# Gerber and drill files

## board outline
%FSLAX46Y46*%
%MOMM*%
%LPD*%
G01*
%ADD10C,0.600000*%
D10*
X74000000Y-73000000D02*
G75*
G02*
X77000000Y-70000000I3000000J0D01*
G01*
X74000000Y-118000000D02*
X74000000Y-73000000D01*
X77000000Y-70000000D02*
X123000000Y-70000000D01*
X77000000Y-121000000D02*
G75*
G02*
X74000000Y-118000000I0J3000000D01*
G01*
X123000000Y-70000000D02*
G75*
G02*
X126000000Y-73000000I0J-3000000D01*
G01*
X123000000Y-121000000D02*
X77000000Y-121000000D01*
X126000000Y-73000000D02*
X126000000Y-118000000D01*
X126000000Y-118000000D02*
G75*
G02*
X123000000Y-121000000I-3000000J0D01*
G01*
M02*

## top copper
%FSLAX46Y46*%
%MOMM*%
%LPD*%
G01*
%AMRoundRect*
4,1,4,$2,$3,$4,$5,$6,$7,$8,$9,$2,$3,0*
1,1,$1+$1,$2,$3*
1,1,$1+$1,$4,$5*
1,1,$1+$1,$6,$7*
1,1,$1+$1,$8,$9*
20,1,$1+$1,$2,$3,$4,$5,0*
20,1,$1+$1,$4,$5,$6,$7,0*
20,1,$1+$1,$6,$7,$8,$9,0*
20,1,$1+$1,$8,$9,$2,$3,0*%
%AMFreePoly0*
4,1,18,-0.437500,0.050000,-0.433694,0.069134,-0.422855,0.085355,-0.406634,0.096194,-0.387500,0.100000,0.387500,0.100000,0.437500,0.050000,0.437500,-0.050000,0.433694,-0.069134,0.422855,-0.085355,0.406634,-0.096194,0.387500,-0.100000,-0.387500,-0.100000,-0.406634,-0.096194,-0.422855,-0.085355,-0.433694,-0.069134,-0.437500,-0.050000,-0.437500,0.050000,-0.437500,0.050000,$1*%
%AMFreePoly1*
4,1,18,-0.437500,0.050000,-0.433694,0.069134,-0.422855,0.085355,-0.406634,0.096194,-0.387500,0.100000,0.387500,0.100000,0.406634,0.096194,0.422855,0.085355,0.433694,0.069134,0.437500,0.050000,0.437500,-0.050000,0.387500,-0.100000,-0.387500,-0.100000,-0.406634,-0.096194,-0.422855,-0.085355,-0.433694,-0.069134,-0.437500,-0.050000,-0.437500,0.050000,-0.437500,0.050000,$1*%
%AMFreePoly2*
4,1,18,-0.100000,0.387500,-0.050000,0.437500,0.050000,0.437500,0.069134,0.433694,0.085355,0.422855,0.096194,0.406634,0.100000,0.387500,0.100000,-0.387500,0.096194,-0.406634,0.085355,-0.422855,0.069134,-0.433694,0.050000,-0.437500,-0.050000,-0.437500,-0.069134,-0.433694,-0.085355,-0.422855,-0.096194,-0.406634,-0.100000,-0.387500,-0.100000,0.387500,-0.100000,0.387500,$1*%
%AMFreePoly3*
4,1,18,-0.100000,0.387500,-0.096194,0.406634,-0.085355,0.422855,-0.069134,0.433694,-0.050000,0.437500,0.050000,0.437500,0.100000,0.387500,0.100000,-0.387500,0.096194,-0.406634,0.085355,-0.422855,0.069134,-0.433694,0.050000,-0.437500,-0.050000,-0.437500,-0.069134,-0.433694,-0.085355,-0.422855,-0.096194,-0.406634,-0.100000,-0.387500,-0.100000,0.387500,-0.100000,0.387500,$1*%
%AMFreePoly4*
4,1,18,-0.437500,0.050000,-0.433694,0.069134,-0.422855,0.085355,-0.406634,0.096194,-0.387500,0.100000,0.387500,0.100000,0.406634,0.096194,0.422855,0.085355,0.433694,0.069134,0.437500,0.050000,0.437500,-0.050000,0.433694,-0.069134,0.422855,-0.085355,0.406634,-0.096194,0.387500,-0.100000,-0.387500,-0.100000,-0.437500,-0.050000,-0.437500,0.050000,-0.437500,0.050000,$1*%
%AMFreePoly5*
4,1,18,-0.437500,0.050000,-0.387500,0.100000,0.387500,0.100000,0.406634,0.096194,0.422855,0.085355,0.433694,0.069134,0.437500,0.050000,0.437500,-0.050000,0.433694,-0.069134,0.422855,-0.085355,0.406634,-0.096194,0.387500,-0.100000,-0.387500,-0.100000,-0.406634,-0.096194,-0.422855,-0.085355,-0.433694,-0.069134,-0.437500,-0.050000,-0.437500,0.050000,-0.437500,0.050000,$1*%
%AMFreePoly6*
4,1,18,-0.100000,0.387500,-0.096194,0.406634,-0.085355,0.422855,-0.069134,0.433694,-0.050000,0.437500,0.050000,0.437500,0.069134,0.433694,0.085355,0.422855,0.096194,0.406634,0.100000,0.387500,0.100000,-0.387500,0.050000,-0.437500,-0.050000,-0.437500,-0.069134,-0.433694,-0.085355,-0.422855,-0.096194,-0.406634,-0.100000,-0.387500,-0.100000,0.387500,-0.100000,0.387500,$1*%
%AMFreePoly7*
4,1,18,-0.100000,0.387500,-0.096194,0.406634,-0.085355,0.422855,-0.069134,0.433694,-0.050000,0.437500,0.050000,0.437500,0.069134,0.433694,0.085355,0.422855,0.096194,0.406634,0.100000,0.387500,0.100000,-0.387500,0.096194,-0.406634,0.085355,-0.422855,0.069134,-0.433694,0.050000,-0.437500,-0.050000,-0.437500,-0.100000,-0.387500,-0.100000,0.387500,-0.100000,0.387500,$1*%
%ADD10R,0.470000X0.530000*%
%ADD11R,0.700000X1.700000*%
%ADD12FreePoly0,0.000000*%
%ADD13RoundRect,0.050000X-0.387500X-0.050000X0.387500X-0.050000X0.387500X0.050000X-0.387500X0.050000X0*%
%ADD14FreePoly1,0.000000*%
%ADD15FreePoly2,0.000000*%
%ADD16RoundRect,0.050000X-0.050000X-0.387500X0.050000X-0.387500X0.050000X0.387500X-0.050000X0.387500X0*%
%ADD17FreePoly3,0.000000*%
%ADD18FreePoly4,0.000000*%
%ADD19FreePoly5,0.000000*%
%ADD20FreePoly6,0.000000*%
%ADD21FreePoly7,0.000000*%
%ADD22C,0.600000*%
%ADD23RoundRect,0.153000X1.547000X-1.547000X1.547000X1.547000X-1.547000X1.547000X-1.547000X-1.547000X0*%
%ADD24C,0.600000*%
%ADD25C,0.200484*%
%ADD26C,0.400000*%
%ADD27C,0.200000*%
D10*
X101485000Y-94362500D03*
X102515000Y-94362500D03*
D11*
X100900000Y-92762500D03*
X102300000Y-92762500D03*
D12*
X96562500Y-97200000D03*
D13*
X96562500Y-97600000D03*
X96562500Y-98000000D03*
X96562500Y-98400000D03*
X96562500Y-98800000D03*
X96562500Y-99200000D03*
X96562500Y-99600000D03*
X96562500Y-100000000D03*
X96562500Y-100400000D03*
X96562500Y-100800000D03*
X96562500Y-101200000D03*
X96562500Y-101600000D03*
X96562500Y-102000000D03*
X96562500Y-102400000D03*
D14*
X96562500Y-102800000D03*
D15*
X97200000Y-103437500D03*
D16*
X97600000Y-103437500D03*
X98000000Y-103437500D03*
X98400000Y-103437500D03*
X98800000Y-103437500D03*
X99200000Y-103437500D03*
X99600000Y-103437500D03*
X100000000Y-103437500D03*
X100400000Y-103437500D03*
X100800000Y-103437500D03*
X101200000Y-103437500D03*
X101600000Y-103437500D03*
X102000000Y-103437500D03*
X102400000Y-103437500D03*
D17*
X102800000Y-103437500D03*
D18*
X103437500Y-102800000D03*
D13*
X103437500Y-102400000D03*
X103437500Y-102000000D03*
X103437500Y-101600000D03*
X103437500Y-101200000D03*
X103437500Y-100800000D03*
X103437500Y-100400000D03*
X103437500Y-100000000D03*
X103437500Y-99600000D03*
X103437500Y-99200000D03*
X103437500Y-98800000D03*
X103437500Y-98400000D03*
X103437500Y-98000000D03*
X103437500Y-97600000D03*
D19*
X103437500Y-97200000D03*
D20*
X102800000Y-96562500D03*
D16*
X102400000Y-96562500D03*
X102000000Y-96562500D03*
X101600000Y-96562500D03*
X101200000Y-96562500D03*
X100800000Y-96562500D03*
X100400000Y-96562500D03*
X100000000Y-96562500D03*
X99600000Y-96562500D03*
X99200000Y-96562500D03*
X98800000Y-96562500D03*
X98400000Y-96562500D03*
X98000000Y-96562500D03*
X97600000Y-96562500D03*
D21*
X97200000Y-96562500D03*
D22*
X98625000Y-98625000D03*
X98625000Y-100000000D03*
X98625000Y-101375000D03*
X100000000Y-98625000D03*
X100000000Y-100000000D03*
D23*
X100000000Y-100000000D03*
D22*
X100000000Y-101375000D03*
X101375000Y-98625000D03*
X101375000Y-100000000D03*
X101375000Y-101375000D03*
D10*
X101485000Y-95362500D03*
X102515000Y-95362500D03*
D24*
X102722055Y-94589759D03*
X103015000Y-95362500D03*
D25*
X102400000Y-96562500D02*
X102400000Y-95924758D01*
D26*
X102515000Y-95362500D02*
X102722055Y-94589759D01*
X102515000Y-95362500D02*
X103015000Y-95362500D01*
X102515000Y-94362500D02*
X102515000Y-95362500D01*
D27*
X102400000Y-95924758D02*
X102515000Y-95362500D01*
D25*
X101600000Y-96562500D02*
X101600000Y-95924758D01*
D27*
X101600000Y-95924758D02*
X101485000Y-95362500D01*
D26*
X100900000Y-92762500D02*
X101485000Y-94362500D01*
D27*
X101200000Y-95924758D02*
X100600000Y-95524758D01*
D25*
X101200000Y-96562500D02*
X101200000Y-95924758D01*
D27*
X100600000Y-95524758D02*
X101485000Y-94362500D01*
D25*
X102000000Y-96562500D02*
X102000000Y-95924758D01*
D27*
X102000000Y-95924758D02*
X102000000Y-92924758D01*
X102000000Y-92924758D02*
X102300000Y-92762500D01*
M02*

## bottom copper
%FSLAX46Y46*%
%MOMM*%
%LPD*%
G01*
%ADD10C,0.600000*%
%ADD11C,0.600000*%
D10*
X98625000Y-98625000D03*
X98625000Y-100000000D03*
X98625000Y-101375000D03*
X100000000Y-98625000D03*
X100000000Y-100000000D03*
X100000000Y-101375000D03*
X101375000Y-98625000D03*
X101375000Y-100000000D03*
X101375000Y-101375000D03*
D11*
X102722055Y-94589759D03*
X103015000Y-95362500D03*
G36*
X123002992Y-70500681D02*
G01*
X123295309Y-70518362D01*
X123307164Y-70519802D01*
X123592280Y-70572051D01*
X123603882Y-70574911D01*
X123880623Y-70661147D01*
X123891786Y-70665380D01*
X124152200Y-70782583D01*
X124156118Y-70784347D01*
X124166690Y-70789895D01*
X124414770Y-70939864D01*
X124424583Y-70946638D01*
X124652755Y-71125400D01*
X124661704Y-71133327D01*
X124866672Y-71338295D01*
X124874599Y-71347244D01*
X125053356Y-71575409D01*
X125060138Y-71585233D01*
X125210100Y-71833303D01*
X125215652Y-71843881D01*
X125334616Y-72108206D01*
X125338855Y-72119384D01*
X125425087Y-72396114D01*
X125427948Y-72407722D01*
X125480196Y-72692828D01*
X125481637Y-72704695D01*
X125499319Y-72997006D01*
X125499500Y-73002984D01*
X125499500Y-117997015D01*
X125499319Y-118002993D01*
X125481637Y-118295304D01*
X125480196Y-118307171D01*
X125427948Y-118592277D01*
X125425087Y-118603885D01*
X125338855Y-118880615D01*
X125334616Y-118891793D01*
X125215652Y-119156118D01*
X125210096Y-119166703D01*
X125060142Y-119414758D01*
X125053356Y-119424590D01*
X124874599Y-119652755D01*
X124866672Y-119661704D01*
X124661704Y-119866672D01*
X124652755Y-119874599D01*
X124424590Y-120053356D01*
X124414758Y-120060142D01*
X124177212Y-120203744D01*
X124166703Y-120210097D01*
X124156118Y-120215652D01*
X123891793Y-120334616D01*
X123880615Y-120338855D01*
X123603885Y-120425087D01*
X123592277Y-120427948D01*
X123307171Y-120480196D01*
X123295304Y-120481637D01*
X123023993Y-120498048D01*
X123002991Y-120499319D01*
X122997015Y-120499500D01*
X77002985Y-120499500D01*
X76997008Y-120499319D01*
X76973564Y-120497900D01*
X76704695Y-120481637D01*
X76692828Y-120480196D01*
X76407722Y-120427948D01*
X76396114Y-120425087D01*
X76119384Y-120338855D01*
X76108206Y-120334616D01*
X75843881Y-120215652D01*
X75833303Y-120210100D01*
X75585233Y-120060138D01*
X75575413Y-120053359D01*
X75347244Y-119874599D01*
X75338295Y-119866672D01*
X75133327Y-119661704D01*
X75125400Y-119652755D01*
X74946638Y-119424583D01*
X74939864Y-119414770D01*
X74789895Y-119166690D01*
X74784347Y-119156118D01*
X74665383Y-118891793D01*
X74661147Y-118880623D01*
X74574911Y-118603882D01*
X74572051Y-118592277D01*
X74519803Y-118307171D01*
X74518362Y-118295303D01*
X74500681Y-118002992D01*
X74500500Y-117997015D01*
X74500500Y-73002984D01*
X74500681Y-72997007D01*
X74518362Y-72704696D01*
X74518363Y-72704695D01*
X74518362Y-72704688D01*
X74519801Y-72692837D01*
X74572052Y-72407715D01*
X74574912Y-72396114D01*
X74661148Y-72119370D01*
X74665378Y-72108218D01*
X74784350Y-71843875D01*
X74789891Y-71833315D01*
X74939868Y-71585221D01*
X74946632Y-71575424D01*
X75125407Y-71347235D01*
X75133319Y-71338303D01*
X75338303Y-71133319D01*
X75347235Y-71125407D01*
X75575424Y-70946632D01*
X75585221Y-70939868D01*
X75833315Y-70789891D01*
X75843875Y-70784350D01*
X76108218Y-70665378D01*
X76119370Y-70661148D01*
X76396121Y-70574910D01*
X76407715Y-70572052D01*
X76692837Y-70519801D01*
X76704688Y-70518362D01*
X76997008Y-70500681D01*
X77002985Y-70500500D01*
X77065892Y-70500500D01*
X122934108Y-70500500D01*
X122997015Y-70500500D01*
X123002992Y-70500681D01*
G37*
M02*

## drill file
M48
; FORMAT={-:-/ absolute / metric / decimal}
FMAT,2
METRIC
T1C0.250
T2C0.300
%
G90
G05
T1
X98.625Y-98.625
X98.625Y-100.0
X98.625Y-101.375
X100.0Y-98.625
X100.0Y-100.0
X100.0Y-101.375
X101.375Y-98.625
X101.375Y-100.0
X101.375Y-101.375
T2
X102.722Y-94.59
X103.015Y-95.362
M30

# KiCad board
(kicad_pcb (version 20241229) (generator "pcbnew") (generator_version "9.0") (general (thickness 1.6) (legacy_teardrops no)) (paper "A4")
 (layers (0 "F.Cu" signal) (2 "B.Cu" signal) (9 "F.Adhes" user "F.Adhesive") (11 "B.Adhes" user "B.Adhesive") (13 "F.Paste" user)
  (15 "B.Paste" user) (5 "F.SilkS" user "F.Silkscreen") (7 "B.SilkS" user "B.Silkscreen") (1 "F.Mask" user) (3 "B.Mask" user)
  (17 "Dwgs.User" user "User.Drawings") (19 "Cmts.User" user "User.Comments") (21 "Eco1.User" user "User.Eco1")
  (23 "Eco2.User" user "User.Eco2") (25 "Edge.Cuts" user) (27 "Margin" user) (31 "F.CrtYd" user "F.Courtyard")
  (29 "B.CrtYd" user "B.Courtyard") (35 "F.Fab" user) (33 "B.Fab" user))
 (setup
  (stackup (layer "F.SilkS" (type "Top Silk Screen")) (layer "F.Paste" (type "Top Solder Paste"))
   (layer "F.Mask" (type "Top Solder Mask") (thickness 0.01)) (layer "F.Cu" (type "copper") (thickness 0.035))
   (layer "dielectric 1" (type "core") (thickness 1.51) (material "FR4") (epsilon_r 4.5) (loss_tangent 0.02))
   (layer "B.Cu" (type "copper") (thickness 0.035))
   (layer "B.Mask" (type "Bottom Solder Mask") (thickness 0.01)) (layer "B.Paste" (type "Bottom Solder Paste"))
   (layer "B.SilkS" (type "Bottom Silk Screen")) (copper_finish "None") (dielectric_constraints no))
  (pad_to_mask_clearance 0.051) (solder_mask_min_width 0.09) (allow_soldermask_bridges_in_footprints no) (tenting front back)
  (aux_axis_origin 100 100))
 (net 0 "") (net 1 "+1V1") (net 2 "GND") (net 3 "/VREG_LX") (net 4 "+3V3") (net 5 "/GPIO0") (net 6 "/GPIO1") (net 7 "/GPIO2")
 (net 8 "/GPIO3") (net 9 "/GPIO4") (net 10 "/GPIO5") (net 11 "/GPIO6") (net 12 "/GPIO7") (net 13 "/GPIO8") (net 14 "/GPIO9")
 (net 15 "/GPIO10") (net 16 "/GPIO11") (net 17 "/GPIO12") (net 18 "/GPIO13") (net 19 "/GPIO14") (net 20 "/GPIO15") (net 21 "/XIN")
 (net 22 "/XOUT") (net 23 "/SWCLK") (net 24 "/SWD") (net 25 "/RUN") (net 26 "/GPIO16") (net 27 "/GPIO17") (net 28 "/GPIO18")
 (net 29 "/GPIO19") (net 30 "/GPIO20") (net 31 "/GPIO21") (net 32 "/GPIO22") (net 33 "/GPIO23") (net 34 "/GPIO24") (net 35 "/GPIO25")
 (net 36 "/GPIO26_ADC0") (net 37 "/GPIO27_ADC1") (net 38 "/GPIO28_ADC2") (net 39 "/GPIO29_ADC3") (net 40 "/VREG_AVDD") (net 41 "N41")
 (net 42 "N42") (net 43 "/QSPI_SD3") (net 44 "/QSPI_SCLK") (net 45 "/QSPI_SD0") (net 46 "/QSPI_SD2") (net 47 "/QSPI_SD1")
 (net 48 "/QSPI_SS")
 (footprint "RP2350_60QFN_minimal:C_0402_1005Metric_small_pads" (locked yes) (layer "F.Cu") (at 102 94.3625)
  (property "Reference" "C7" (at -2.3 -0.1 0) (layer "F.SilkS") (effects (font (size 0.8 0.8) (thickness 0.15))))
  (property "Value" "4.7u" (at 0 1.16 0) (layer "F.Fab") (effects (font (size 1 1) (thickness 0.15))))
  (pad "1" smd rect (at -0.515 0) (size 0.47 0.53) (layers "F.Cu" "F.Mask" "F.Paste") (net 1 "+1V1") (clearance 0.125))
  (pad "2" smd rect (at 0.515 0) (size 0.47 0.53) (layers "F.Cu" "F.Mask" "F.Paste") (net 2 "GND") (clearance 0.125)))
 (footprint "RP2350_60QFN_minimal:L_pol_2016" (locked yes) (layer "F.Cu") (at 101.6 92.7625)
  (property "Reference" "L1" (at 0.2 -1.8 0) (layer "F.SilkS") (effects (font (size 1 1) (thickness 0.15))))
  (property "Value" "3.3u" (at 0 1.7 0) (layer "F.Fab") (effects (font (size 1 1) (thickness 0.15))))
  (pad "1" smd rect (at -0.7 0) (size 0.7 1.7) (layers "F.Cu" "F.Mask" "F.Paste") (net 1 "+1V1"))
  (pad "2" smd rect (at 0.7 0) (size 0.7 1.7) (layers "F.Cu" "F.Mask" "F.Paste") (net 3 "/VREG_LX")))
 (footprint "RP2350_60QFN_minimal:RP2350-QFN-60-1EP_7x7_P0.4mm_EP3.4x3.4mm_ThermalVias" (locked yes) (layer "F.Cu") (at 100 100)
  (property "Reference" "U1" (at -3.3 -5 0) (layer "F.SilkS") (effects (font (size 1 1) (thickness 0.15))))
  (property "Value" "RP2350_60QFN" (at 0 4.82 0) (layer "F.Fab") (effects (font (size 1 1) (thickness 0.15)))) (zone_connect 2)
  (pad "" smd roundrect (at -0.7 -0.7) (size 1.2 1.2) (layers "F.Paste") (roundrect_rratio 0.2083333333) (zone_connect 2))
  (pad "" smd roundrect (at -0.7 0.7) (size 1.2 1.2) (layers "F.Paste") (roundrect_rratio 0.2083333333) (zone_connect 2))
  (pad "" smd roundrect (at 0.7 -0.7) (size 1.2 1.2) (layers "F.Paste") (roundrect_rratio 0.2083333333) (zone_connect 2))
  (pad "" smd roundrect (at 0.7 0.7) (size 1.2 1.2) (layers "F.Paste") (roundrect_rratio 0.2083333333) (zone_connect 2))
  (pad "1" smd roundrect (at -3.4375 -2.8) (size 0.875 0.2) (layers "F.Cu" "F.Mask" "F.Paste") (roundrect_rratio 0.25) (chamfer_ratio 0.25)
   (chamfer top_right) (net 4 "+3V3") (zone_connect 2))
  (pad "2" smd roundrect (at -3.4375 -2.4) (size 0.875 0.2) (layers "F.Cu" "F.Mask" "F.Paste") (roundrect_rratio 0.25) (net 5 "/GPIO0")
   (zone_connect 2))
  (pad "3" smd roundrect (at -3.4375 -2) (size 0.875 0.2) (layers "F.Cu" "F.Mask" "F.Paste") (roundrect_rratio 0.25) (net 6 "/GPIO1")
   (zone_connect 2))
  (pad "4" smd roundrect (at -3.4375 -1.6) (size 0.875 0.2) (layers "F.Cu" "F.Mask" "F.Paste") (roundrect_rratio 0.25) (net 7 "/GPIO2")
   (zone_connect 2))
  (pad "5" smd roundrect (at -3.4375 -1.2) (size 0.875 0.2) (layers "F.Cu" "F.Mask" "F.Paste") (roundrect_rratio 0.25) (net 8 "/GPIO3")
   (zone_connect 2))
  (pad "6" smd roundrect (at -3.4375 -0.8) (size 0.875 0.2) (layers "F.Cu" "F.Mask" "F.Paste") (roundrect_rratio 0.25) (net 1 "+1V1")
   (zone_connect 2))
  (pad "7" smd roundrect (at -3.4375 -0.4) (size 0.875 0.2) (layers "F.Cu" "F.Mask" "F.Paste") (roundrect_rratio 0.25) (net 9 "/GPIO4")
   (zone_connect 2))
  (pad "8" smd roundrect (at -3.4375 0) (size 0.875 0.2) (layers "F.Cu" "F.Mask" "F.Paste") (roundrect_rratio 0.25) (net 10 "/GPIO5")
   (zone_connect 2))
  (pad "9" smd roundrect (at -3.4375 0.4) (size 0.875 0.2) (layers "F.Cu" "F.Mask" "F.Paste") (roundrect_rratio 0.25) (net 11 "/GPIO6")
   (zone_connect 2))
  (pad "10" smd roundrect (at -3.4375 0.8) (size 0.875 0.2) (layers "F.Cu" "F.Mask" "F.Paste") (roundrect_rratio 0.25) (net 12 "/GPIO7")
   (zone_connect 2))
  (pad "11" smd roundrect (at -3.4375 1.2) (size 0.875 0.2) (layers "F.Cu" "F.Mask" "F.Paste") (roundrect_rratio 0.25) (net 4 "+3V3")
   (zone_connect 2))
  (pad "12" smd roundrect (at -3.4375 1.6) (size 0.875 0.2) (layers "F.Cu" "F.Mask" "F.Paste") (roundrect_rratio 0.25) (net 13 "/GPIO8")
   (zone_connect 2))
  (pad "13" smd roundrect (at -3.4375 2) (size 0.875 0.2) (layers "F.Cu" "F.Mask" "F.Paste") (roundrect_rratio 0.25) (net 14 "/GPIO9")
   (zone_connect 2))
  (pad "14" smd roundrect (at -3.4375 2.4) (size 0.875 0.2) (layers "F.Cu" "F.Mask" "F.Paste") (roundrect_rratio 0.25) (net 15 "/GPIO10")
   (zone_connect 2))
  (pad "15" smd roundrect (at -3.4375 2.8) (size 0.875 0.2) (layers "F.Cu" "F.Mask" "F.Paste") (roundrect_rratio 0.25) (chamfer_ratio 0.25)
   (chamfer bottom_right) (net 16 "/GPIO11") (zone_connect 2))
  (pad "16" smd roundrect (at -2.8 3.4375) (size 0.2 0.875) (layers "F.Cu" "F.Mask" "F.Paste") (roundrect_rratio 0.25) (chamfer_ratio 0.25)
   (chamfer top_left) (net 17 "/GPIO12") (zone_connect 2))
  (pad "17" smd roundrect (at -2.4 3.4375) (size 0.2 0.875) (layers "F.Cu" "F.Mask" "F.Paste") (roundrect_rratio 0.25) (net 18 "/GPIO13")
   (zone_connect 2))
  (pad "18" smd roundrect (at -2 3.4375) (size 0.2 0.875) (layers "F.Cu" "F.Mask" "F.Paste") (roundrect_rratio 0.25) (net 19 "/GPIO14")
   (zone_connect 2))
  (pad "19" smd roundrect (at -1.6 3.4375) (size 0.2 0.875) (layers "F.Cu" "F.Mask" "F.Paste") (roundrect_rratio 0.25) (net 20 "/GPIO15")
   (zone_connect 2))
  (pad "20" smd roundrect (at -1.2 3.4375) (size 0.2 0.875) (layers "F.Cu" "F.Mask" "F.Paste") (roundrect_rratio 0.25) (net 4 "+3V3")
   (zone_connect 2))
  (pad "21" smd roundrect (at -0.8 3.4375) (size 0.2 0.875) (layers "F.Cu" "F.Mask" "F.Paste") (roundrect_rratio 0.25) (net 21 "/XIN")
   (zone_connect 2))
  (pad "22" smd roundrect (at -0.4 3.4375) (size 0.2 0.875) (layers "F.Cu" "F.Mask" "F.Paste") (roundrect_rratio 0.25) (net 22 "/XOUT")
   (zone_connect 2))
  (pad "23" smd roundrect (at 0 3.4375) (size 0.2 0.875) (layers "F.Cu" "F.Mask" "F.Paste") (roundrect_rratio 0.25) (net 1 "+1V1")
   (zone_connect 2))
  (pad "24" smd roundrect (at 0.4 3.4375) (size 0.2 0.875) (layers "F.Cu" "F.Mask" "F.Paste") (roundrect_rratio 0.25) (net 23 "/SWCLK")
   (zone_connect 2))
  (pad "25" smd roundrect (at 0.8 3.4375) (size 0.2 0.875) (layers "F.Cu" "F.Mask" "F.Paste") (roundrect_rratio 0.25) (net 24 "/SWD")
   (zone_connect 2))
  (pad "26" smd roundrect (at 1.2 3.4375) (size 0.2 0.875) (layers "F.Cu" "F.Mask" "F.Paste") (roundrect_rratio 0.25) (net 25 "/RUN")
   (zone_connect 2))
  (pad "27" smd roundrect (at 1.6 3.4375) (size 0.2 0.875) (layers "F.Cu" "F.Mask" "F.Paste") (roundrect_rratio 0.25) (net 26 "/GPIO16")
   (zone_connect 2))
  (pad "28" smd roundrect (at 2 3.4375) (size 0.2 0.875) (layers "F.Cu" "F.Mask" "F.Paste") (roundrect_rratio 0.25) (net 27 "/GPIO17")
   (zone_connect 2))
  (pad "29" smd roundrect (at 2.4 3.4375) (size 0.2 0.875) (layers "F.Cu" "F.Mask" "F.Paste") (roundrect_rratio 0.25) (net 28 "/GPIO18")
   (zone_connect 2))
  (pad "30" smd roundrect (at 2.8 3.4375) (size 0.2 0.875) (layers "F.Cu" "F.Mask" "F.Paste") (roundrect_rratio 0.25) (chamfer_ratio 0.25)
   (chamfer top_right) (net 4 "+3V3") (zone_connect 2))
  (pad "31" smd roundrect (at 3.4375 2.8) (size 0.875 0.2) (layers "F.Cu" "F.Mask" "F.Paste") (roundrect_rratio 0.25) (chamfer_ratio 0.25)
   (chamfer bottom_left) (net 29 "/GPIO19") (zone_connect 2))
  (pad "32" smd roundrect (at 3.4375 2.4) (size 0.875 0.2) (layers "F.Cu" "F.Mask" "F.Paste") (roundrect_rratio 0.25) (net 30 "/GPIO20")
   (zone_connect 2))
  (pad "33" smd roundrect (at 3.4375 2) (size 0.875 0.2) (layers "F.Cu" "F.Mask" "F.Paste") (roundrect_rratio 0.25) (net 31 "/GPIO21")
   (zone_connect 2))
  (pad "34" smd roundrect (at 3.4375 1.6) (size 0.875 0.2) (layers "F.Cu" "F.Mask" "F.Paste") (roundrect_rratio 0.25) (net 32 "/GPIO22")
   (zone_connect 2))
  (pad "35" smd roundrect (at 3.4375 1.2) (size 0.875 0.2) (layers "F.Cu" "F.Mask" "F.Paste") (roundrect_rratio 0.25) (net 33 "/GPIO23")
   (zone_connect 2))
  (pad "36" smd roundrect (at 3.4375 0.8) (size 0.875 0.2) (layers "F.Cu" "F.Mask" "F.Paste") (roundrect_rratio 0.25) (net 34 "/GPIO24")
   (zone_connect 2))
  (pad "37" smd roundrect (at 3.4375 0.4) (size 0.875 0.2) (layers "F.Cu" "F.Mask" "F.Paste") (roundrect_rratio 0.25) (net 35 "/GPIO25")
   (zone_connect 2))
  (pad "38" smd roundrect (at 3.4375 0) (size 0.875 0.2) (layers "F.Cu" "F.Mask" "F.Paste") (roundrect_rratio 0.25) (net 4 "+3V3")
   (zone_connect 2))
  (pad "39" smd roundrect (at 3.4375 -0.4) (size 0.875 0.2) (layers "F.Cu" "F.Mask" "F.Paste") (roundrect_rratio 0.25) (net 1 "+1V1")
   (zone_connect 2))
  (pad "40" smd roundrect (at 3.4375 -0.8) (size 0.875 0.2) (layers "F.Cu" "F.Mask" "F.Paste") (roundrect_rratio 0.25)
   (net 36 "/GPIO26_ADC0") (zone_connect 2))
  (pad "41" smd roundrect (at 3.4375 -1.2) (size 0.875 0.2) (layers "F.Cu" "F.Mask" "F.Paste") (roundrect_rratio 0.25)
   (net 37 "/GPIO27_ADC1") (zone_connect 2))
  (pad "42" smd roundrect (at 3.4375 -1.6) (size 0.875 0.2) (layers "F.Cu" "F.Mask" "F.Paste") (roundrect_rratio 0.25)
   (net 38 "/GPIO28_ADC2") (zone_connect 2))
  (pad "43" smd roundrect (at 3.4375 -2) (size 0.875 0.2) (layers "F.Cu" "F.Mask" "F.Paste") (roundrect_rratio 0.25) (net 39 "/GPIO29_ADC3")
   (zone_connect 2))
  (pad "44" smd roundrect (at 3.4375 -2.4) (size 0.875 0.2) (layers "F.Cu" "F.Mask" "F.Paste") (roundrect_rratio 0.25) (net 4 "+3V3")
   (zone_connect 2))
  (pad "45" smd roundrect (at 3.4375 -2.8) (size 0.875 0.2) (layers "F.Cu" "F.Mask" "F.Paste") (roundrect_rratio 0.25) (chamfer_ratio 0.25)
   (chamfer top_left) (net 4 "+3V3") (zone_connect 2))
  (pad "46" smd roundrect (at 2.8 -3.4375) (size 0.2 0.875) (layers "F.Cu" "F.Mask" "F.Paste") (roundrect_rratio 0.25) (chamfer_ratio 0.25)
   (chamfer bottom_right) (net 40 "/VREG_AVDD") (zone_connect 2))
  (pad "47" smd roundrect (at 2.4 -3.4375) (size 0.2 0.875) (layers "F.Cu" "F.Mask" "F.Paste") (roundrect_rratio 0.25) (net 2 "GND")
   (zone_connect 2))
  (pad "48" smd roundrect (at 2 -3.4375) (size 0.2 0.875) (layers "F.Cu" "F.Mask" "F.Paste") (roundrect_rratio 0.25) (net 3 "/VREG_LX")
   (zone_connect 2))
  (pad "49" smd roundrect (at 1.6 -3.4375) (size 0.2 0.875) (layers "F.Cu" "F.Mask" "F.Paste") (roundrect_rratio 0.25) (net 4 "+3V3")
   (zone_connect 2))
  (pad "50" smd roundrect (at 1.2 -3.4375) (size 0.2 0.875) (layers "F.Cu" "F.Mask" "F.Paste") (roundrect_rratio 0.25) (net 1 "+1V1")
   (zone_connect 2))
  (pad "51" smd roundrect (at 0.8 -3.4375) (size 0.2 0.875) (layers "F.Cu" "F.Mask" "F.Paste") (roundrect_rratio 0.25) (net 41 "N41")
   (zone_connect 2))
  (pad "52" smd roundrect (at 0.4 -3.4375) (size 0.2 0.875) (layers "F.Cu" "F.Mask" "F.Paste") (roundrect_rratio 0.25) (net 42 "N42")
   (zone_connect 2))
  (pad "53" smd roundrect (at 0 -3.4375) (size 0.2 0.875) (layers "F.Cu" "F.Mask" "F.Paste") (roundrect_rratio 0.25) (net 4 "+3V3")
   (zone_connect 2))
  (pad "54" smd roundrect (at -0.4 -3.4375) (size 0.2 0.875) (layers "F.Cu" "F.Mask" "F.Paste") (roundrect_rratio 0.25) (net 4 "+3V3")
   (zone_connect 2))
  (pad "55" smd roundrect (at -0.8 -3.4375) (size 0.2 0.875) (layers "F.Cu" "F.Mask" "F.Paste") (roundrect_rratio 0.25) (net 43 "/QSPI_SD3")
   (zone_connect 2))
  (pad "56" smd roundrect (at -1.2 -3.4375) (size 0.2 0.875) (layers "F.Cu" "F.Mask" "F.Paste") (roundrect_rratio 0.25)
   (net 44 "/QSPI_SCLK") (zone_connect 2))
  (pad "57" smd roundrect (at -1.6 -3.4375) (size 0.2 0.875) (layers "F.Cu" "F.Mask" "F.Paste") (roundrect_rratio 0.25) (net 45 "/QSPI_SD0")
   (zone_connect 2))
  (pad "58" smd roundrect (at -2 -3.4375) (size 0.2 0.875) (layers "F.Cu" "F.Mask" "F.Paste") (roundrect_rratio 0.25) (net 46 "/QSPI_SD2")
   (zone_connect 2))
  (pad "59" smd roundrect (at -2.4 -3.4375) (size 0.2 0.875) (layers "F.Cu" "F.Mask" "F.Paste") (roundrect_rratio 0.25) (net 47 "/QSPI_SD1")
   (zone_connect 2))
  (pad "60" smd roundrect (at -2.8 -3.4375) (size 0.2 0.875) (layers "F.Cu" "F.Mask" "F.Paste") (roundrect_rratio 0.25) (chamfer_ratio 0.25)
   (chamfer bottom_left) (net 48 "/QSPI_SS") (zone_connect 2))
  (pad "61" thru_hole circle (at -1.375 -1.375) (size 0.6 0.6) (drill 0.25) (layers "*.Cu") (remove_unused_layers no) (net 2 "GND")
   (zone_connect 2))
  (pad "61" thru_hole circle (at -1.375 0) (size 0.6 0.6) (drill 0.25) (layers "*.Cu") (remove_unused_layers no) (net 2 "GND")
   (zone_connect 2))
  (pad "61" thru_hole circle (at -1.375 1.375) (size 0.6 0.6) (drill 0.25) (layers "*.Cu") (remove_unused_layers no) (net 2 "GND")
   (zone_connect 2))
  (pad "61" thru_hole circle (at 0 -1.375) (size 0.6 0.6) (drill 0.25) (layers "*.Cu") (remove_unused_layers no) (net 2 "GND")
   (zone_connect 2))
  (pad "61" thru_hole circle (at 0 0) (size 0.6 0.6) (drill 0.25) (layers "*.Cu") (remove_unused_layers no) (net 2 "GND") (zone_connect 2))
  (pad "61" smd roundrect (at 0 0 90) (size 3.4 3.4) (layers "F.Cu" "F.Mask") (roundrect_rratio 0.045) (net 2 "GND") (zone_connect 2))
  (pad "61" thru_hole circle (at 0 1.375) (size 0.6 0.6) (drill 0.25) (layers "*.Cu") (remove_unused_layers no) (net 2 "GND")
   (zone_connect 2))
  (pad "61" thru_hole circle (at 1.375 -1.375) (size 0.6 0.6) (drill 0.25) (layers "*.Cu") (remove_unused_layers no) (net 2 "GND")
   (zone_connect 2))
  (pad "61" thru_hole circle (at 1.375 0) (size 0.6 0.6) (drill 0.25) (layers "*.Cu") (remove_unused_layers no) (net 2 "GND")
   (zone_connect 2))
  (pad "61" thru_hole circle (at 1.375 1.375) (size 0.6 0.6) (drill 0.25) (layers "*.Cu") (remove_unused_layers no) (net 2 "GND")
   (zone_connect 2)))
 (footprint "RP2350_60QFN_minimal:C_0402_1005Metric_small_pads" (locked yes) (layer "F.Cu") (at 102 95.3625)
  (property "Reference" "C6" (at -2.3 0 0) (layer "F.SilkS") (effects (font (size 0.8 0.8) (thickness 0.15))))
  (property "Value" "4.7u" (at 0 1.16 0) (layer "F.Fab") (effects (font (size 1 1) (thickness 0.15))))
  (pad "1" smd rect (at -0.515 0) (size 0.47 0.53) (layers "F.Cu" "F.Mask" "F.Paste") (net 4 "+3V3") (clearance 0.125))
  (pad "2" smd rect (at 0.515 0) (size 0.47 0.53) (layers "F.Cu" "F.Mask" "F.Paste") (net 2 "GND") (clearance 0.125)))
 (gr_arc (start 74 73) (mid 74.87868 70.87868) (end 77 70) (stroke (width 0.6) (type solid)) (layer "Edge.Cuts"))
 (gr_line (start 74 118) (end 74 73) (stroke (width 0.6) (type solid)) (layer "Edge.Cuts"))
 (gr_line (start 77 70) (end 123 70) (stroke (width 0.6) (type solid)) (layer "Edge.Cuts"))
 (gr_arc (start 77 121) (mid 74.87868 120.12132) (end 74 118) (stroke (width 0.6) (type solid)) (layer "Edge.Cuts"))
 (gr_arc (start 123 70) (mid 125.12132 70.87868) (end 126 73) (stroke (width 0.6) (type solid)) (layer "Edge.Cuts"))
 (gr_line (start 123 121) (end 77 121) (stroke (width 0.6) (type solid)) (layer "Edge.Cuts"))
 (gr_line (start 126 73) (end 126 118) (stroke (width 0.6) (type solid)) (layer "Edge.Cuts"))
 (gr_arc (start 126 118) (mid 125.12132 120.12132) (end 123 121) (stroke (width 0.6) (type solid)) (layer "Edge.Cuts"))
 (segment (start 102.4 96.5625) (end 102.4 95.924758) (width 0.200484) (locked yes) (layer "F.Cu") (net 2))
 (segment (start 102.515 95.3625) (end 102.722055 94.589759) (width 0.4) (locked yes) (layer "F.Cu") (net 2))
 (segment (start 102.515 95.3625) (end 103.015 95.3625) (width 0.4) (locked yes) (layer "F.Cu") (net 2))
 (segment (start 102.515 94.3625) (end 102.515 95.3625) (width 0.4) (locked yes) (layer "F.Cu") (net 2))
 (segment (start 102.4 95.924758) (end 102.515 95.3625) (width 0.2) (locked yes) (layer "F.Cu") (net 2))
 (via (at 102.722055 94.589759) (size 0.6) (drill 0.3) (layers "F.Cu" "B.Cu") (locked yes) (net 2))
 (via (at 103.015 95.3625) (size 0.6) (drill 0.3) (layers "F.Cu" "B.Cu") (locked yes) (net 2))
 (segment (start 101.6 96.5625) (end 101.6 95.924758) (width 0.200484) (locked yes) (layer "F.Cu") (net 4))
 (segment (start 101.6 95.924758) (end 101.485 95.3625) (width 0.2) (locked yes) (layer "F.Cu") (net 4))
 (segment (start 100.9 92.7625) (end 101.485 94.3625) (width 0.4) (locked yes) (layer "F.Cu") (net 1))
 (segment (start 101.2 95.924758) (end 100.6 95.524758) (width 0.2) (locked yes) (layer "F.Cu") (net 1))
 (segment (start 101.2 96.5625) (end 101.2 95.924758) (width 0.200484) (locked yes) (layer "F.Cu") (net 1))
 (segment (start 100.6 95.524758) (end 101.485 94.3625) (width 0.2) (locked yes) (layer "F.Cu") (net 1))
 (segment (start 102 96.5625) (end 102 95.924758) (width 0.200484) (locked yes) (layer "F.Cu") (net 3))
 (segment (start 102 95.924758) (end 102 92.924758) (width 0.2) (locked yes) (layer "F.Cu") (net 3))
 (segment (start 102 92.924758) (end 102.3 92.7625) (width 0.2) (locked yes) (layer "F.Cu") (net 3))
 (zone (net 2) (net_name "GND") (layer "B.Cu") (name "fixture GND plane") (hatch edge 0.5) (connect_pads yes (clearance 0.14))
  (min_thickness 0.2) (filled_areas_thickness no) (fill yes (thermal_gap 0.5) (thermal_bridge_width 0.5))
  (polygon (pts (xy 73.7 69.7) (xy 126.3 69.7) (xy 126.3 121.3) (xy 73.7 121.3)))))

